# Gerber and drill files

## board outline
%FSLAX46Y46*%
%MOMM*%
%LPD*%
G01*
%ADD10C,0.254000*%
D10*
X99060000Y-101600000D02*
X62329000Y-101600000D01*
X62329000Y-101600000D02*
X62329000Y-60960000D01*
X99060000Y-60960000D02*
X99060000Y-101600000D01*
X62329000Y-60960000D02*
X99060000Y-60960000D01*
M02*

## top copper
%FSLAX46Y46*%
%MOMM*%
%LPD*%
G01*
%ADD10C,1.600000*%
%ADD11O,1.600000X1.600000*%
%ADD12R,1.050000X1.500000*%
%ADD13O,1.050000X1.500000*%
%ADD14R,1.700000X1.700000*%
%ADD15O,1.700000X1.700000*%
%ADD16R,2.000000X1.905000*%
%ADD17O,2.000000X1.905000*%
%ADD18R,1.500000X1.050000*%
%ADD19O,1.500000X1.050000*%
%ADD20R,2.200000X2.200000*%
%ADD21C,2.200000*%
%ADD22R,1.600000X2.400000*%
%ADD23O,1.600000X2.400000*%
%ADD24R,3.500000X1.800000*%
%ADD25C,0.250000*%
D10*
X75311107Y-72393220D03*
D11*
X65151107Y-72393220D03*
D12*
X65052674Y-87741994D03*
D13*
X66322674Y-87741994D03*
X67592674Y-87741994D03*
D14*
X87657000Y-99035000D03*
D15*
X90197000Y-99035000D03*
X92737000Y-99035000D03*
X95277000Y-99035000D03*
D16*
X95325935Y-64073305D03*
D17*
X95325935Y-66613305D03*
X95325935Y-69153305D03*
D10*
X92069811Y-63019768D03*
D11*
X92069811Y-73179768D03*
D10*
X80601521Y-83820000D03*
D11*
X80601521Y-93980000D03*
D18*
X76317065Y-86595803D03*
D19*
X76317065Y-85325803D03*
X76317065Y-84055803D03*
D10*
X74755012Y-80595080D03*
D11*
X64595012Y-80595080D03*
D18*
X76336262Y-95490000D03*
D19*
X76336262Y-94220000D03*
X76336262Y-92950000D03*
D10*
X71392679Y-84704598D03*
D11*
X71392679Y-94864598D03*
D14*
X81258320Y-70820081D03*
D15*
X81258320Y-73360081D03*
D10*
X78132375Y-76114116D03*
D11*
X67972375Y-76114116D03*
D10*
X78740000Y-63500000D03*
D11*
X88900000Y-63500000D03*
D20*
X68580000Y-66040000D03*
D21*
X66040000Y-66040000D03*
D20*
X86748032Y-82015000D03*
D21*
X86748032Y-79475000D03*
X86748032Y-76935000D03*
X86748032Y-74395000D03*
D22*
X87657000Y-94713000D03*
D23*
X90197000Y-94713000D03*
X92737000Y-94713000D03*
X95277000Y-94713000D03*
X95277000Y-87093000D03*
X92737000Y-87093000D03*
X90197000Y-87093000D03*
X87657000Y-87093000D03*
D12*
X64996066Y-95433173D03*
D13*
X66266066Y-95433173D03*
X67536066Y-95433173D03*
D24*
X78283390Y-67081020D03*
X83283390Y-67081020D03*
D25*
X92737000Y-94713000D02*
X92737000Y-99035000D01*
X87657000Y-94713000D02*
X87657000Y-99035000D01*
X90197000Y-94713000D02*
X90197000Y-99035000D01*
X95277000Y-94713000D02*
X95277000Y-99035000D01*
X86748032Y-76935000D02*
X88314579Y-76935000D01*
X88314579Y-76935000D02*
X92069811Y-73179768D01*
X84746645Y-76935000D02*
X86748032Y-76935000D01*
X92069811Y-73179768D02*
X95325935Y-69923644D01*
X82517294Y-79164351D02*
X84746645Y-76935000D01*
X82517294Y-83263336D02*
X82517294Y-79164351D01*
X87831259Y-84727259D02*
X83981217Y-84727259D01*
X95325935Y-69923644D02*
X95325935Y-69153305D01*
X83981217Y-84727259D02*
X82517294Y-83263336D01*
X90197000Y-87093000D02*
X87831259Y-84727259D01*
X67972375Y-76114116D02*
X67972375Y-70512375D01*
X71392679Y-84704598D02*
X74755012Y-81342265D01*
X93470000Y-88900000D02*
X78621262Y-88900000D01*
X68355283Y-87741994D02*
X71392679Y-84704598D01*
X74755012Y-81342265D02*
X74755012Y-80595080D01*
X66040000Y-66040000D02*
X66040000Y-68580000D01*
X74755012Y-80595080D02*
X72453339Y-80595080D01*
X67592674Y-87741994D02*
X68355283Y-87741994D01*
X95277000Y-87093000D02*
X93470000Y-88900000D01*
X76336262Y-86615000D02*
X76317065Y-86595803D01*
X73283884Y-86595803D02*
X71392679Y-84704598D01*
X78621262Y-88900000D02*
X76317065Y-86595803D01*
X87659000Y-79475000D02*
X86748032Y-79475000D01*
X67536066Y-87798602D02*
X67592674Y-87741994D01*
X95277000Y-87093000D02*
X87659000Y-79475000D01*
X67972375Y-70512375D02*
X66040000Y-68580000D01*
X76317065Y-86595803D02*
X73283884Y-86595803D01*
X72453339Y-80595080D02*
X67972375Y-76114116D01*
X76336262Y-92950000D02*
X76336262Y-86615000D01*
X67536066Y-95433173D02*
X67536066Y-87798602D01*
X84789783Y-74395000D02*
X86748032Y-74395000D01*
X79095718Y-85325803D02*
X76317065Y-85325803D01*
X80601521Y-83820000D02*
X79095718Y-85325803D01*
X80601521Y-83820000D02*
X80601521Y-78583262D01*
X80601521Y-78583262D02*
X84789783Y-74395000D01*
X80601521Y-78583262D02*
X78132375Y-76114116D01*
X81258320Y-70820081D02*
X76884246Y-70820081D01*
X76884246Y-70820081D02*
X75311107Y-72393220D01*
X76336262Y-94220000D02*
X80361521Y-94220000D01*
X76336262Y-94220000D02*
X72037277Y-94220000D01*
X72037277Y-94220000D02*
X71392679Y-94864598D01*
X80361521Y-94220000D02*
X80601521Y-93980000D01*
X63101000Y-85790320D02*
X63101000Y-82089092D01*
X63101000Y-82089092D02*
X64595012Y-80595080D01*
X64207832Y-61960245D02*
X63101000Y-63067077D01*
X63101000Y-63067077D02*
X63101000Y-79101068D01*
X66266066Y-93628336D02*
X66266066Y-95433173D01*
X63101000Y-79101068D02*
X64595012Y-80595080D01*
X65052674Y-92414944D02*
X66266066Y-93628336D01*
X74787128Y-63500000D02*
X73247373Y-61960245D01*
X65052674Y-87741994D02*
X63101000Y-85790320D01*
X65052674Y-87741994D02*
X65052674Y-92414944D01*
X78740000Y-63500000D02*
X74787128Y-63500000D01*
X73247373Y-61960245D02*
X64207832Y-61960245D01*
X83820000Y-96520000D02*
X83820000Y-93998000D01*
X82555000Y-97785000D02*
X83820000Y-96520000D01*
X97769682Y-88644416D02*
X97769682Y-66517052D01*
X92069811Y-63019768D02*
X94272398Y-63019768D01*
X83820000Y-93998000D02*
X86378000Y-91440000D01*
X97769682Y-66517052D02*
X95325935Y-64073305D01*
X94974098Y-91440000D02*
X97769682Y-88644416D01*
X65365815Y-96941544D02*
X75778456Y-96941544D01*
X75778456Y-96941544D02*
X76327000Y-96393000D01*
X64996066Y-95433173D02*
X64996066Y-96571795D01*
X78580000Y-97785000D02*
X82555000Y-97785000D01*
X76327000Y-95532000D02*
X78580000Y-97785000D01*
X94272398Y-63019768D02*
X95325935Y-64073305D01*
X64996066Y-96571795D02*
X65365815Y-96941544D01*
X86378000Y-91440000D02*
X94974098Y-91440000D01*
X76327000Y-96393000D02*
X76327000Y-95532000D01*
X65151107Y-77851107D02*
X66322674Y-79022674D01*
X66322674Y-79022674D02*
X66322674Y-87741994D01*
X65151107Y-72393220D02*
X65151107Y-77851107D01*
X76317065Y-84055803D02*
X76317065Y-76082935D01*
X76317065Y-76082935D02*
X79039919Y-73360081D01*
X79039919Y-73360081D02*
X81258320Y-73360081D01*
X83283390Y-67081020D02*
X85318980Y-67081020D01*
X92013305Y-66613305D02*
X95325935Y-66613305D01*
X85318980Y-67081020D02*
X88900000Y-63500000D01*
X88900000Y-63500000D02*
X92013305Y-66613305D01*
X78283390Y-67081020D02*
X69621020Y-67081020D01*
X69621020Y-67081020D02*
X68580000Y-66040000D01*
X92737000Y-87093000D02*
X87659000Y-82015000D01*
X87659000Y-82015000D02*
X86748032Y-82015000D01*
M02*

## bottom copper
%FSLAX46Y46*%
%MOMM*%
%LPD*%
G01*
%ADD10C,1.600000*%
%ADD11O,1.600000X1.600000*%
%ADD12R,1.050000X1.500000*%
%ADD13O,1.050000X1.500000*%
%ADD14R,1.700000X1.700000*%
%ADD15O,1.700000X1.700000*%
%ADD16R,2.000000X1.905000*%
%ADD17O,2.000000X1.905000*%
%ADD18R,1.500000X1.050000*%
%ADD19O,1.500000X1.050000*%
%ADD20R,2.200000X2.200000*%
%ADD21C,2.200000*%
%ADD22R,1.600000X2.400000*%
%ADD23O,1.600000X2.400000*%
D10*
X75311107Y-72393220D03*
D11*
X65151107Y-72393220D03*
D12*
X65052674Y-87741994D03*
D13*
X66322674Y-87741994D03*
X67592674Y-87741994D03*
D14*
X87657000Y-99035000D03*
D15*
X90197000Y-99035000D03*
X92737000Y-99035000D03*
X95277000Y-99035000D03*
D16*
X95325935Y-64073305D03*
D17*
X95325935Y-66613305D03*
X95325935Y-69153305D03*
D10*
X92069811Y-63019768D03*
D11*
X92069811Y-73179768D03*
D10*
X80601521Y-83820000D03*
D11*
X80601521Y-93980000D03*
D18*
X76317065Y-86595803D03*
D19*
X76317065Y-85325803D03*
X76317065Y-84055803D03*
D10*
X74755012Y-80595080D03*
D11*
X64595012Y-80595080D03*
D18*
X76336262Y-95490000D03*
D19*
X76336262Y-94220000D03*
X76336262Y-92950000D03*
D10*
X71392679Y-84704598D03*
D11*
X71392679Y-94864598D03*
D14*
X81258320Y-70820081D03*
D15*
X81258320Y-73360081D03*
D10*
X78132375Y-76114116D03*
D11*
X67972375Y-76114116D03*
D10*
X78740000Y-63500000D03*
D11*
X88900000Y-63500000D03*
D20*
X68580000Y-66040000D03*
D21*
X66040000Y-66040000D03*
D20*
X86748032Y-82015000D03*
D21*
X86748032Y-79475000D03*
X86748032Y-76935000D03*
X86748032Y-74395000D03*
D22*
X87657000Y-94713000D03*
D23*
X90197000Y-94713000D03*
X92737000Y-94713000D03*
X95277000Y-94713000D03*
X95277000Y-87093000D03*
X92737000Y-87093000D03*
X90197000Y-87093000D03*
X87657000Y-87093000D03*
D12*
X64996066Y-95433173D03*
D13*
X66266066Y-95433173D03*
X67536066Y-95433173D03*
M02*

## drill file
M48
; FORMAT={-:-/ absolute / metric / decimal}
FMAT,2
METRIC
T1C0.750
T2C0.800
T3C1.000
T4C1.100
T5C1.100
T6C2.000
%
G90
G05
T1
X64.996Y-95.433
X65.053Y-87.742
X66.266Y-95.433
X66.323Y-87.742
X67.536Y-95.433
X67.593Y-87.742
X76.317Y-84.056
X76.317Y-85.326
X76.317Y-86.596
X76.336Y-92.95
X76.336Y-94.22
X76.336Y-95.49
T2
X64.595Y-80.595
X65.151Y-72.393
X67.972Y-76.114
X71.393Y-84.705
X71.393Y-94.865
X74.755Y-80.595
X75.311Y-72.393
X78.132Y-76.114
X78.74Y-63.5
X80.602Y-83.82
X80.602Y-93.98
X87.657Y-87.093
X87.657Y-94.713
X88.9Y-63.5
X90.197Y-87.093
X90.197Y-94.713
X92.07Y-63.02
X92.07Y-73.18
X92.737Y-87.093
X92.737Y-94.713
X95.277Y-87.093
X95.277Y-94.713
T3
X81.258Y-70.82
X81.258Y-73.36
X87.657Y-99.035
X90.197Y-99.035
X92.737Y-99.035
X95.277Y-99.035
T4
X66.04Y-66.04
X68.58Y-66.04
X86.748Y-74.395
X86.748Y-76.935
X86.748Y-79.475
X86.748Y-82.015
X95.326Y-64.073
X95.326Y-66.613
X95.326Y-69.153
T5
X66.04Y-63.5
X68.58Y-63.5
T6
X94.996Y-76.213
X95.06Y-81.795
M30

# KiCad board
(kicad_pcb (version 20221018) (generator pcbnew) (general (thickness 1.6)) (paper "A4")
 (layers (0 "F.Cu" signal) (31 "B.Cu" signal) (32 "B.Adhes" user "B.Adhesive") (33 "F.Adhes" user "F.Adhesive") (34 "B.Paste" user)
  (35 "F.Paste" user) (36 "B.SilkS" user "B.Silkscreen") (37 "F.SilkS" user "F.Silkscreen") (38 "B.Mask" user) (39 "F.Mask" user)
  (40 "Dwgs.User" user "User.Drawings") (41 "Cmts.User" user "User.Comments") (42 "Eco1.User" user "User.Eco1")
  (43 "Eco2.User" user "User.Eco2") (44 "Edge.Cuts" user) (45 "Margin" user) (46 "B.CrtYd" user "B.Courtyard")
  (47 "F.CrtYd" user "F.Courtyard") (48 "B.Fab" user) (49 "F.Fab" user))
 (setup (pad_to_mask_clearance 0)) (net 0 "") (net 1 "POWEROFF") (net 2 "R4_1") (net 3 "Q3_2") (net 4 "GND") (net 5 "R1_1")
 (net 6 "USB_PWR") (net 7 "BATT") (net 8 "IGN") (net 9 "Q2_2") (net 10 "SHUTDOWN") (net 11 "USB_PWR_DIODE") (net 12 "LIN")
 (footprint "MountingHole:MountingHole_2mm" (layer "F.Cu") (at 94.99557 76.212882)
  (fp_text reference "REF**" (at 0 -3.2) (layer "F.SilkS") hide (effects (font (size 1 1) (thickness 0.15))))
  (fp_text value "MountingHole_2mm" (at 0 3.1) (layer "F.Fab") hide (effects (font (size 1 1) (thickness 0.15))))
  (pad "" np_thru_hole circle (at 0 0) (size 2 2) (drill 2) (layers "*.Cu" "*.Mask")))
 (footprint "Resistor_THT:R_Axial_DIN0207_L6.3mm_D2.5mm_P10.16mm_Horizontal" (layer "F.Cu") (at 75.311107 72.39322 180)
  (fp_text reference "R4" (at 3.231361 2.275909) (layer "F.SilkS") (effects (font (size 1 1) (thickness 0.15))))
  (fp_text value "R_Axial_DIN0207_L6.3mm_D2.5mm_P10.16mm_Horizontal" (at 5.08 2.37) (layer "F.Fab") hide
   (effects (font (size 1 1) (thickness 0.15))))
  (pad "1" thru_hole circle (at 0 0 180) (size 1.6 1.6) (drill 0.8) (layers "*.Cu" "*.Mask") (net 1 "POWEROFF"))
  (pad "2" thru_hole oval (at 10.16 0 180) (size 1.6 1.6) (drill 0.8) (layers "*.Cu" "*.Mask") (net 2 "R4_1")))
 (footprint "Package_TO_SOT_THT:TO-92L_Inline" (layer "F.Cu") (at 65.052674 87.741994)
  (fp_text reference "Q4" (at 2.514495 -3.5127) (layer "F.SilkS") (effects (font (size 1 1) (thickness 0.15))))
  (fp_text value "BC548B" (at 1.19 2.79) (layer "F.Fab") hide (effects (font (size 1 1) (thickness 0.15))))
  (pad "1" thru_hole rect (at 0 0) (size 1.05 1.5) (drill 0.75) (layers "*.Cu" "*.Mask") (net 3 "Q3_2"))
  (pad "2" thru_hole oval (at 1.27 0) (size 1.05 1.5) (drill 0.75) (layers "*.Cu" "*.Mask") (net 2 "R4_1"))
  (pad "3" thru_hole oval (at 2.54 0) (size 1.05 1.5) (drill 0.75) (layers "*.Cu" "*.Mask") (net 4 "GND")))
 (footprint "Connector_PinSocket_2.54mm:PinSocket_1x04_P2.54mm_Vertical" (layer "F.Cu") (at 87.657 99.035 90)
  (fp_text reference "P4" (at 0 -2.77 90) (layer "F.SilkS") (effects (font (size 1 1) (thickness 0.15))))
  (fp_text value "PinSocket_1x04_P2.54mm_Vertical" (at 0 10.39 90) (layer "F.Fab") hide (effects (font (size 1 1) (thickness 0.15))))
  (pad "1" thru_hole rect (at 0 0 90) (size 1.7 1.7) (drill 1) (layers "*.Cu" "*.Mask"))
  (pad "2" thru_hole oval (at 0 2.54 90) (size 1.7 1.7) (drill 1) (layers "*.Cu" "*.Mask"))
  (pad "3" thru_hole oval (at 0 5.08 90) (size 1.7 1.7) (drill 1) (layers "*.Cu" "*.Mask"))
  (pad "4" thru_hole oval (at 0 7.62 90) (size 1.7 1.7) (drill 1) (layers "*.Cu" "*.Mask")))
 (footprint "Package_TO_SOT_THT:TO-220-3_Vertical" (layer "F.Cu") (at 95.325935 64.073305 -90)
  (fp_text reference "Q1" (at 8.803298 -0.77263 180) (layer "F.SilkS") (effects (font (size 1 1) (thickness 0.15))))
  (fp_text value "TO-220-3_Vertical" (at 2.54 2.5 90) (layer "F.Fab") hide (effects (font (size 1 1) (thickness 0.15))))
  (pad "1" thru_hole rect (at 0 0 270) (size 1.905 2) (drill 1.1) (layers "*.Cu" "*.Mask") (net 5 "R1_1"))
  (pad "2" thru_hole oval (at 2.54 0 270) (size 1.905 2) (drill 1.1) (layers "*.Cu" "*.Mask") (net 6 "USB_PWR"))
  (pad "3" thru_hole oval (at 5.08 0 270) (size 1.905 2) (drill 1.1) (layers "*.Cu" "*.Mask") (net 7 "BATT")))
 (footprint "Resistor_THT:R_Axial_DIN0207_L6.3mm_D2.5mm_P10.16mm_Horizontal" (layer "F.Cu") (at 92.069811 63.019768 -90)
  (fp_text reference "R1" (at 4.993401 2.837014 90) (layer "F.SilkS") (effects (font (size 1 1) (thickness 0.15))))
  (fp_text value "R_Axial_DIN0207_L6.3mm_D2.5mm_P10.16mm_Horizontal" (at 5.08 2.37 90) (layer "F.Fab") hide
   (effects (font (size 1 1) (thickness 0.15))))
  (pad "1" thru_hole circle (at 0 0 270) (size 1.6 1.6) (drill 0.8) (layers "*.Cu" "*.Mask") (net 5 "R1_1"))
  (pad "2" thru_hole oval (at 10.16 0 270) (size 1.6 1.6) (drill 0.8) (layers "*.Cu" "*.Mask") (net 7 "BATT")))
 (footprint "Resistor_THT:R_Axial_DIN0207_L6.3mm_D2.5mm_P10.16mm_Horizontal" (layer "F.Cu") (at 80.601521 83.82 -90)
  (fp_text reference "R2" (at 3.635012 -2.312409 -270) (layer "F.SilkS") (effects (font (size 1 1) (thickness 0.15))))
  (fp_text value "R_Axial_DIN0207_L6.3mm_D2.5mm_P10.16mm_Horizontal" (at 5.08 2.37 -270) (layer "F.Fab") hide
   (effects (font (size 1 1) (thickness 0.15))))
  (pad "1" thru_hole circle (at 0 0 270) (size 1.6 1.6) (drill 0.8) (layers "*.Cu" "*.Mask") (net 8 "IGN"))
  (pad "2" thru_hole oval (at 10.16 0 270) (size 1.6 1.6) (drill 0.8) (layers "*.Cu" "*.Mask") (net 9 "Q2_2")))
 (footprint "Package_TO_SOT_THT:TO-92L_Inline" (layer "F.Cu") (at 76.317065 86.595803 90)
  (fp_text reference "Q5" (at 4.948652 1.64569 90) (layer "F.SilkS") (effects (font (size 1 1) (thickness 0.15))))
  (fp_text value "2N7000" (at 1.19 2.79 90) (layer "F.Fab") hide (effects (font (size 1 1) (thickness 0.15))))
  (pad "1" thru_hole rect (at 0 0 90) (size 1.05 1.5) (drill 0.75) (layers "*.Cu" "*.Mask") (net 4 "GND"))
  (pad "2" thru_hole oval (at 1.27 0 90) (size 1.05 1.5) (drill 0.75) (layers "*.Cu" "*.Mask") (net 8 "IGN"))
  (pad "3" thru_hole oval (at 2.54 0 90) (size 1.05 1.5) (drill 0.75) (layers "*.Cu" "*.Mask") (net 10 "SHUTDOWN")))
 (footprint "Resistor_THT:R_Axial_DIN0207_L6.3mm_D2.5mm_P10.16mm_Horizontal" (layer "F.Cu") (at 74.755012 80.59508 180)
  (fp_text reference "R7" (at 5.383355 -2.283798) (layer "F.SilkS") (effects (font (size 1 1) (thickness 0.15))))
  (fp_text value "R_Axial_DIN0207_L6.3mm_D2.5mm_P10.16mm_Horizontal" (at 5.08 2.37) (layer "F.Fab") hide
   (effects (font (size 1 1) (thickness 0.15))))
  (pad "1" thru_hole circle (at 0 0 180) (size 1.6 1.6) (drill 0.8) (layers "*.Cu" "*.Mask") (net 4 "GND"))
  (pad "2" thru_hole oval (at 10.16 0 180) (size 1.6 1.6) (drill 0.8) (layers "*.Cu" "*.Mask") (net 3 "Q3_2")))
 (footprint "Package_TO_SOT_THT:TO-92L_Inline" (layer "F.Cu") (at 76.336262 95.49 90)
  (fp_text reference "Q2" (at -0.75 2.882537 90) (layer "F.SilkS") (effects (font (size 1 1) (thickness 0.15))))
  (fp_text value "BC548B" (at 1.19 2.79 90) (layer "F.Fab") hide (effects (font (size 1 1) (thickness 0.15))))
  (pad "1" thru_hole rect (at 0 0 90) (size 1.05 1.5) (drill 0.75) (layers "*.Cu" "*.Mask") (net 5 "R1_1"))
  (pad "2" thru_hole oval (at 1.27 0 90) (size 1.05 1.5) (drill 0.75) (layers "*.Cu" "*.Mask") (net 9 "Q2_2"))
  (pad "3" thru_hole oval (at 2.54 0 90) (size 1.05 1.5) (drill 0.75) (layers "*.Cu" "*.Mask") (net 4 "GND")))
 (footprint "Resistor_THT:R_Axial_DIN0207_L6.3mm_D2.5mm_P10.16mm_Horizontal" (layer "F.Cu") (at 71.392679 84.704598 -90)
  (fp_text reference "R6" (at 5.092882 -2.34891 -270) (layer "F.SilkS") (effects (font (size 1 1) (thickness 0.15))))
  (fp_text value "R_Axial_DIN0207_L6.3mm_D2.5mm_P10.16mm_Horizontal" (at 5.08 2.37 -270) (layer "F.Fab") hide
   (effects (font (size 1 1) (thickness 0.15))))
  (pad "1" thru_hole circle (at 0 0 270) (size 1.6 1.6) (drill 0.8) (layers "*.Cu" "*.Mask") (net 4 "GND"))
  (pad "2" thru_hole oval (at 10.16 0 270) (size 1.6 1.6) (drill 0.8) (layers "*.Cu" "*.Mask") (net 9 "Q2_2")))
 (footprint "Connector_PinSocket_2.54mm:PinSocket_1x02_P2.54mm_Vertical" (layer "F.Cu") (at 81.25832 70.820081)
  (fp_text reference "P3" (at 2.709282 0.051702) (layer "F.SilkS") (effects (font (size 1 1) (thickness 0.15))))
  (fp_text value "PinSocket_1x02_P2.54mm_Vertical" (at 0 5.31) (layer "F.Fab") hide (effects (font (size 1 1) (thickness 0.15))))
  (pad "1" thru_hole rect (at 0 0) (size 1.7 1.7) (drill 1) (layers "*.Cu" "*.Mask") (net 1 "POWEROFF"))
  (pad "2" thru_hole oval (at 0 2.54) (size 1.7 1.7) (drill 1) (layers "*.Cu" "*.Mask") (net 10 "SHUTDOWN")))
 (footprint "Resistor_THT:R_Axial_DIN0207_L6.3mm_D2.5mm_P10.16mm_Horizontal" (layer "F.Cu") (at 78.132375 76.114116 180)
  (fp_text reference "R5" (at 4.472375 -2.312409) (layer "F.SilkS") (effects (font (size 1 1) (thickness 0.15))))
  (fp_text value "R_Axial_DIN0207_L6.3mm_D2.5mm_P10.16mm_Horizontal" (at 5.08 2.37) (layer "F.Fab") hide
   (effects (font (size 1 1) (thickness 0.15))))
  (pad "1" thru_hole circle (at 0 0 180) (size 1.6 1.6) (drill 0.8) (layers "*.Cu" "*.Mask") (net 8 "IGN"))
  (pad "2" thru_hole oval (at 10.16 0 180) (size 1.6 1.6) (drill 0.8) (layers "*.Cu" "*.Mask") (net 4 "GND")))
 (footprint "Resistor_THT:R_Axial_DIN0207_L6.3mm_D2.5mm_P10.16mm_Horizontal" (layer "F.Cu") (at 78.74 63.5)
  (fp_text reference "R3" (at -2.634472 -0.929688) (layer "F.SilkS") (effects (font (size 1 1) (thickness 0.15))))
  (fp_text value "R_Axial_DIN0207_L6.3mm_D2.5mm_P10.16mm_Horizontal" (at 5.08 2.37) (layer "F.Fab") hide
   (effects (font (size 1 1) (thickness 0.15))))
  (pad "1" thru_hole circle (at 0 0) (size 1.6 1.6) (drill 0.8) (layers "*.Cu" "*.Mask") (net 3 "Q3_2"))
  (pad "2" thru_hole oval (at 10.16 0) (size 1.6 1.6) (drill 0.8) (layers "*.Cu" "*.Mask") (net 6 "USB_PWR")))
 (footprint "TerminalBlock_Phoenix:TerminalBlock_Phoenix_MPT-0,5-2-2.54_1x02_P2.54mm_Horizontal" (layer "F.Cu") (at 68.58 66.04 180)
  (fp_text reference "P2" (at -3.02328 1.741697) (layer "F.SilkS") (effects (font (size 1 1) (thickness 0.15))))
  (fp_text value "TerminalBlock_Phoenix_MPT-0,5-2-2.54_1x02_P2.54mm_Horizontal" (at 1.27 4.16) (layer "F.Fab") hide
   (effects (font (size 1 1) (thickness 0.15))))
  (pad "" np_thru_hole circle (at 0 2.54 180) (size 1.1 1.1) (drill 1.1) (layers "*.Cu" "*.Mask"))
  (pad "" np_thru_hole circle (at 2.54 2.54 180) (size 1.1 1.1) (drill 1.1) (layers "*.Cu" "*.Mask"))
  (pad "1" thru_hole rect (at 0 0 180) (size 2.2 2.2) (drill 1.1) (layers "*.Cu" "*.Mask") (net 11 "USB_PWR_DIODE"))
  (pad "2" thru_hole circle (at 2.54 0 180) (size 2.2 2.2) (drill 1.1) (layers "*.Cu" "*.Mask") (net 4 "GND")))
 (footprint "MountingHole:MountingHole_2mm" (layer "F.Cu") (at 95.059983 81.794719)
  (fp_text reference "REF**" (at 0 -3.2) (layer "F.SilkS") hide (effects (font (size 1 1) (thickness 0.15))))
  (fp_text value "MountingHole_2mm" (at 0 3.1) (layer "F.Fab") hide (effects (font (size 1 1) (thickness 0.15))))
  (pad "" np_thru_hole circle (at 0 0) (size 2 2) (drill 2) (layers "*.Cu" "*.Mask")))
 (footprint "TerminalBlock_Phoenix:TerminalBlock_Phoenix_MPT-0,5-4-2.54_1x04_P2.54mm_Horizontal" (layer "F.Cu") (at 86.748032 82.015 90)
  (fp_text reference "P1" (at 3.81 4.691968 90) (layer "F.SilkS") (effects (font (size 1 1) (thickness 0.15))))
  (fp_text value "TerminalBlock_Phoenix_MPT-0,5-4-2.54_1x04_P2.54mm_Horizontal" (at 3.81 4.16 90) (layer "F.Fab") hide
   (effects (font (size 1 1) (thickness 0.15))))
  (pad "1" thru_hole rect (at 0 0 90) (size 2.2 2.2) (drill 1.1) (layers "*.Cu" "*.Mask") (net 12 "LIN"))
  (pad "2" thru_hole circle (at 2.54 0 90) (size 2.2 2.2) (drill 1.1) (layers "*.Cu" "*.Mask") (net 4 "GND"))
  (pad "3" thru_hole circle (at 5.08 0 90) (size 2.2 2.2) (drill 1.1) (layers "*.Cu" "*.Mask") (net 7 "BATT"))
  (pad "4" thru_hole circle (at 7.62 0 90) (size 2.2 2.2) (drill 1.1) (layers "*.Cu" "*.Mask") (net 8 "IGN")))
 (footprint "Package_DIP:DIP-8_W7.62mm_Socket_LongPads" (layer "F.Cu") (at 87.657 94.713 90)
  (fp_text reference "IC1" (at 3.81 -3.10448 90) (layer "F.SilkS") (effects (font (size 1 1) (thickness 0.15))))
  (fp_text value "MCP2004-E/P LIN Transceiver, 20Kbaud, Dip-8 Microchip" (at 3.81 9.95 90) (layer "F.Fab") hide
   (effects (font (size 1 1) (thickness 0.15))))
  (pad "1" thru_hole rect (at 0 0 90) (size 2.4 1.6) (drill 0.8) (layers "*.Cu" "*.Mask"))
  (pad "2" thru_hole oval (at 0 2.54 90) (size 2.4 1.6) (drill 0.8) (layers "*.Cu" "*.Mask"))
  (pad "3" thru_hole oval (at 0 5.08 90) (size 2.4 1.6) (drill 0.8) (layers "*.Cu" "*.Mask"))
  (pad "4" thru_hole oval (at 0 7.62 90) (size 2.4 1.6) (drill 0.8) (layers "*.Cu" "*.Mask"))
  (pad "5" thru_hole oval (at 7.62 7.62 90) (size 2.4 1.6) (drill 0.8) (layers "*.Cu" "*.Mask") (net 4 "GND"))
  (pad "6" thru_hole oval (at 7.62 5.08 90) (size 2.4 1.6) (drill 0.8) (layers "*.Cu" "*.Mask") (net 12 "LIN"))
  (pad "7" thru_hole oval (at 7.62 2.54 90) (size 2.4 1.6) (drill 0.8) (layers "*.Cu" "*.Mask") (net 7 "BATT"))
  (pad "8" thru_hole oval (at 7.62 0 90) (size 2.4 1.6) (drill 0.8) (layers "*.Cu" "*.Mask")))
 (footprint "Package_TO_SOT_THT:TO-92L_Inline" (layer "F.Cu") (at 64.996066 95.433173)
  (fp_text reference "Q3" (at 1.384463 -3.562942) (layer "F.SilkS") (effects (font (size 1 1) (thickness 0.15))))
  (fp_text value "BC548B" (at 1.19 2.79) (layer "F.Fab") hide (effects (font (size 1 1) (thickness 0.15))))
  (pad "1" thru_hole rect (at 0 0) (size 1.05 1.5) (drill 0.75) (layers "*.Cu" "*.Mask") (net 5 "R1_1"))
  (pad "2" thru_hole oval (at 1.27 0) (size 1.05 1.5) (drill 0.75) (layers "*.Cu" "*.Mask") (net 3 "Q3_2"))
  (pad "3" thru_hole oval (at 2.54 0) (size 1.05 1.5) (drill 0.75) (layers "*.Cu" "*.Mask") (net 4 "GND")))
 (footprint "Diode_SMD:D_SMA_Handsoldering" (layer "F.Cu") (at 80.78339 67.08102)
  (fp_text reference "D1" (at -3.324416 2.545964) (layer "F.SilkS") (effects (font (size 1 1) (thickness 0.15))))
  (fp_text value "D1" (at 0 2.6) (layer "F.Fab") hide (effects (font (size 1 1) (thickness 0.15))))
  (pad "1" smd rect (at -2.5 0) (size 3.5 1.8) (layers "F.Cu" "F.Paste" "F.Mask") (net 11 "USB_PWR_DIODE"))
  (pad "2" smd rect (at 2.5 0) (size 3.5 1.8) (layers "F.Cu" "F.Paste" "F.Mask") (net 6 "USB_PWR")))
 (gr_line (start 99.06 101.6) (end 62.329 101.6) (stroke (width 0.254) (type solid)) (layer "Edge.Cuts"))
 (gr_line (start 62.329 101.6) (end 62.329 60.96) (stroke (width 0.254) (type solid)) (layer "Edge.Cuts"))
 (gr_line (start 99.06 60.96) (end 99.06 101.6) (stroke (width 0.254) (type solid)) (layer "Edge.Cuts"))
 (gr_line (start 62.329 60.96) (end 99.06 60.96) (stroke (width 0.254) (type solid)) (layer "Edge.Cuts"))
 (segment (start 92.737 94.713) (end 92.737 99.035) (width 0.25) (layer "F.Cu") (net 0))
 (segment (start 87.657 94.713) (end 87.657 99.035) (width 0.25) (layer "F.Cu") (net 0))
 (segment (start 90.197 94.713) (end 90.197 99.035) (width 0.25) (layer "F.Cu") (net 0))
 (segment (start 95.277 94.713) (end 95.277 99.035) (width 0.25) (layer "F.Cu") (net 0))
 (segment (start 86.748032 76.935) (end 88.314579 76.935) (width 0.25) (layer "F.Cu") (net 7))
 (segment (start 88.314579 76.935) (end 92.069811 73.179768) (width 0.25) (layer "F.Cu") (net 7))
 (segment (start 84.746645 76.935) (end 86.748032 76.935) (width 0.25) (layer "F.Cu") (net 7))
 (segment (start 92.069811 73.179768) (end 95.325935 69.923644) (width 0.25) (layer "F.Cu") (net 7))
 (segment (start 82.517294 79.164351) (end 84.746645 76.935) (width 0.25) (layer "F.Cu") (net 7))
 (segment (start 82.517294 83.263336) (end 82.517294 79.164351) (width 0.25) (layer "F.Cu") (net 7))
 (segment (start 87.831259 84.727259) (end 83.981217 84.727259) (width 0.25) (layer "F.Cu") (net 7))
 (segment (start 95.325935 69.923644) (end 95.325935 69.153305) (width 0.25) (layer "F.Cu") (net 7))
 (segment (start 83.981217 84.727259) (end 82.517294 83.263336) (width 0.25) (layer "F.Cu") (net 7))
 (segment (start 90.197 87.093) (end 87.831259 84.727259) (width 0.25) (layer "F.Cu") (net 7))
 (segment (start 67.972375 76.114116) (end 67.972375 70.512375) (width 0.25) (layer "F.Cu") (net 4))
 (segment (start 71.392679 84.704598) (end 74.755012 81.342265) (width 0.25) (layer "F.Cu") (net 4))
 (segment (start 93.47 88.9) (end 78.621262 88.9) (width 0.25) (layer "F.Cu") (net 4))
 (segment (start 68.355283 87.741994) (end 71.392679 84.704598) (width 0.25) (layer "F.Cu") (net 4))
 (segment (start 74.755012 81.342265) (end 74.755012 80.59508) (width 0.25) (layer "F.Cu") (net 4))
 (segment (start 66.04 66.04) (end 66.04 68.58) (width 0.25) (layer "F.Cu") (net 4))
 (segment (start 74.755012 80.59508) (end 72.453339 80.59508) (width 0.25) (layer "F.Cu") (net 4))
 (segment (start 67.592674 87.741994) (end 68.355283 87.741994) (width 0.25) (layer "F.Cu") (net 4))
 (segment (start 95.277 87.093) (end 93.47 88.9) (width 0.25) (layer "F.Cu") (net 4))
 (segment (start 76.336262 86.615) (end 76.317065 86.595803) (width 0.25) (layer "F.Cu") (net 4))
 (segment (start 73.283884 86.595803) (end 71.392679 84.704598) (width 0.25) (layer "F.Cu") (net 4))
 (segment (start 78.621262 88.9) (end 76.317065 86.595803) (width 0.25) (layer "F.Cu") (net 4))
 (segment (start 87.659 79.475) (end 86.748032 79.475) (width 0.25) (layer "F.Cu") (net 4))
 (segment (start 67.536066 87.798602) (end 67.592674 87.741994) (width 0.25) (layer "F.Cu") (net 4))
 (segment (start 95.277 87.093) (end 87.659 79.475) (width 0.25) (layer "F.Cu") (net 4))
 (segment (start 67.972375 70.512375) (end 66.04 68.58) (width 0.25) (layer "F.Cu") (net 4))
 (segment (start 76.317065 86.595803) (end 73.283884 86.595803) (width 0.25) (layer "F.Cu") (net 4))
 (segment (start 72.453339 80.59508) (end 67.972375 76.114116) (width 0.25) (layer "F.Cu") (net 4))
 (segment (start 76.336262 92.95) (end 76.336262 86.615) (width 0.25) (layer "F.Cu") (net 4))
 (segment (start 67.536066 95.433173) (end 67.536066 87.798602) (width 0.25) (layer "F.Cu") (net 4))
 (segment (start 84.789783 74.395) (end 86.748032 74.395) (width 0.25) (layer "F.Cu") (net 8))
 (segment (start 79.095718 85.325803) (end 76.317065 85.325803) (width 0.25) (layer "F.Cu") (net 8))
 (segment (start 80.601521 83.82) (end 79.095718 85.325803) (width 0.25) (layer "F.Cu") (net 8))
 (segment (start 80.601521 83.82) (end 80.601521 78.583262) (width 0.25) (layer "F.Cu") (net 8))
 (segment (start 80.601521 78.583262) (end 84.789783 74.395) (width 0.25) (layer "F.Cu") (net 8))
 (segment (start 80.601521 78.583262) (end 78.132375 76.114116) (width 0.25) (layer "F.Cu") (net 8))
 (segment (start 81.25832 70.820081) (end 76.884246 70.820081) (width 0.25) (layer "F.Cu") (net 1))
 (segment (start 76.884246 70.820081) (end 75.311107 72.39322) (width 0.25) (layer "F.Cu") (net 1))
 (segment (start 76.336262 94.22) (end 80.361521 94.22) (width 0.25) (layer "F.Cu") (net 9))
 (segment (start 76.336262 94.22) (end 72.037277 94.22) (width 0.25) (layer "F.Cu") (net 9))
 (segment (start 72.037277 94.22) (end 71.392679 94.864598) (width 0.25) (layer "F.Cu") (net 9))
 (segment (start 80.361521 94.22) (end 80.601521 93.98) (width 0.25) (layer "F.Cu") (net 9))
 (segment (start 63.101 85.79032) (end 63.101 82.089092) (width 0.25) (layer "F.Cu") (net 3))
 (segment (start 63.101 82.089092) (end 64.595012 80.59508) (width 0.25) (layer "F.Cu") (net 3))
 (segment (start 64.207832 61.960245) (end 63.101 63.067077) (width 0.25) (layer "F.Cu") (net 3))
 (segment (start 63.101 63.067077) (end 63.101 79.101068) (width 0.25) (layer "F.Cu") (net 3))
 (segment (start 66.266066 93.628336) (end 66.266066 95.433173) (width 0.25) (layer "F.Cu") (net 3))
 (segment (start 63.101 79.101068) (end 64.595012 80.59508) (width 0.25) (layer "F.Cu") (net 3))
 (segment (start 65.052674 92.414944) (end 66.266066 93.628336) (width 0.25) (layer "F.Cu") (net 3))
 (segment (start 74.787128 63.5) (end 73.247373 61.960245) (width 0.25) (layer "F.Cu") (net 3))
 (segment (start 65.052674 87.741994) (end 63.101 85.79032) (width 0.25) (layer "F.Cu") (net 3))
 (segment (start 65.052674 87.741994) (end 65.052674 92.414944) (width 0.25) (layer "F.Cu") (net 3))
 (segment (start 78.74 63.5) (end 74.787128 63.5) (width 0.25) (layer "F.Cu") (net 3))
 (segment (start 73.247373 61.960245) (end 64.207832 61.960245) (width 0.25) (layer "F.Cu") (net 3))
 (segment (start 83.82 96.52) (end 83.82 93.998) (width 0.25) (layer "F.Cu") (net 5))
 (segment (start 82.555 97.785) (end 83.82 96.52) (width 0.25) (layer "F.Cu") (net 5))
 (segment (start 97.769682 88.644416) (end 97.769682 66.517052) (width 0.25) (layer "F.Cu") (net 5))
 (segment (start 92.069811 63.019768) (end 94.272398 63.019768) (width 0.25) (layer "F.Cu") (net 5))
 (segment (start 83.82 93.998) (end 86.378 91.44) (width 0.25) (layer "F.Cu") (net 5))
 (segment (start 97.769682 66.517052) (end 95.325935 64.073305) (width 0.25) (layer "F.Cu") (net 5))
 (segment (start 94.974098 91.44) (end 97.769682 88.644416) (width 0.25) (layer "F.Cu") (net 5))
 (segment (start 65.365815 96.941544) (end 75.778456 96.941544) (width 0.25) (layer "F.Cu") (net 5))
 (segment (start 75.778456 96.941544) (end 76.327 96.393) (width 0.25) (layer "F.Cu") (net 5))
 (segment (start 64.996066 95.433173) (end 64.996066 96.571795) (width 0.25) (layer "F.Cu") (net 5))
 (segment (start 78.58 97.785) (end 82.555 97.785) (width 0.25) (layer "F.Cu") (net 5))
 (segment (start 76.327 95.532) (end 78.58 97.785) (width 0.25) (layer "F.Cu") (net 5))
 (segment (start 94.272398 63.019768) (end 95.325935 64.073305) (width 0.25) (layer "F.Cu") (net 5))
 (segment (start 64.996066 96.571795) (end 65.365815 96.941544) (width 0.25) (layer "F.Cu") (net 5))
 (segment (start 86.378 91.44) (end 94.974098 91.44) (width 0.25) (layer "F.Cu") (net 5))
 (segment (start 76.327 96.393) (end 76.327 95.532) (width 0.25) (layer "F.Cu") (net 5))
 (segment (start 65.151107 77.851107) (end 66.322674 79.022674) (width 0.25) (layer "F.Cu") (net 2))
 (segment (start 66.322674 79.022674) (end 66.322674 87.741994) (width 0.25) (layer "F.Cu") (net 2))
 (segment (start 65.151107 72.39322) (end 65.151107 77.851107) (width 0.25) (layer "F.Cu") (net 2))
 (segment (start 76.317065 84.055803) (end 76.317065 76.082935) (width 0.25) (layer "F.Cu") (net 10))
 (segment (start 76.317065 76.082935) (end 79.039919 73.360081) (width 0.25) (layer "F.Cu") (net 10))
 (segment (start 79.039919 73.360081) (end 81.25832 73.360081) (width 0.25) (layer "F.Cu") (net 10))
 (segment (start 83.28339 67.08102) (end 85.31898 67.08102) (width 0.25) (layer "F.Cu") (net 6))
 (segment (start 92.013305 66.613305) (end 95.325935 66.613305) (width 0.25) (layer "F.Cu") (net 6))
 (segment (start 85.31898 67.08102) (end 88.9 63.5) (width 0.25) (layer "F.Cu") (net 6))
 (segment (start 88.9 63.5) (end 92.013305 66.613305) (width 0.25) (layer "F.Cu") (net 6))
 (segment (start 78.28339 67.08102) (end 69.62102 67.08102) (width 0.25) (layer "F.Cu") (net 11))
 (segment (start 69.62102 67.08102) (end 68.58 66.04) (width 0.25) (layer "F.Cu") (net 11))
 (segment (start 92.737 87.093) (end 87.659 82.015) (width 0.25) (layer "F.Cu") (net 12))
 (segment (start 87.659 82.015) (end 86.748032 82.015) (width 0.25) (layer "F.Cu") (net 12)))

